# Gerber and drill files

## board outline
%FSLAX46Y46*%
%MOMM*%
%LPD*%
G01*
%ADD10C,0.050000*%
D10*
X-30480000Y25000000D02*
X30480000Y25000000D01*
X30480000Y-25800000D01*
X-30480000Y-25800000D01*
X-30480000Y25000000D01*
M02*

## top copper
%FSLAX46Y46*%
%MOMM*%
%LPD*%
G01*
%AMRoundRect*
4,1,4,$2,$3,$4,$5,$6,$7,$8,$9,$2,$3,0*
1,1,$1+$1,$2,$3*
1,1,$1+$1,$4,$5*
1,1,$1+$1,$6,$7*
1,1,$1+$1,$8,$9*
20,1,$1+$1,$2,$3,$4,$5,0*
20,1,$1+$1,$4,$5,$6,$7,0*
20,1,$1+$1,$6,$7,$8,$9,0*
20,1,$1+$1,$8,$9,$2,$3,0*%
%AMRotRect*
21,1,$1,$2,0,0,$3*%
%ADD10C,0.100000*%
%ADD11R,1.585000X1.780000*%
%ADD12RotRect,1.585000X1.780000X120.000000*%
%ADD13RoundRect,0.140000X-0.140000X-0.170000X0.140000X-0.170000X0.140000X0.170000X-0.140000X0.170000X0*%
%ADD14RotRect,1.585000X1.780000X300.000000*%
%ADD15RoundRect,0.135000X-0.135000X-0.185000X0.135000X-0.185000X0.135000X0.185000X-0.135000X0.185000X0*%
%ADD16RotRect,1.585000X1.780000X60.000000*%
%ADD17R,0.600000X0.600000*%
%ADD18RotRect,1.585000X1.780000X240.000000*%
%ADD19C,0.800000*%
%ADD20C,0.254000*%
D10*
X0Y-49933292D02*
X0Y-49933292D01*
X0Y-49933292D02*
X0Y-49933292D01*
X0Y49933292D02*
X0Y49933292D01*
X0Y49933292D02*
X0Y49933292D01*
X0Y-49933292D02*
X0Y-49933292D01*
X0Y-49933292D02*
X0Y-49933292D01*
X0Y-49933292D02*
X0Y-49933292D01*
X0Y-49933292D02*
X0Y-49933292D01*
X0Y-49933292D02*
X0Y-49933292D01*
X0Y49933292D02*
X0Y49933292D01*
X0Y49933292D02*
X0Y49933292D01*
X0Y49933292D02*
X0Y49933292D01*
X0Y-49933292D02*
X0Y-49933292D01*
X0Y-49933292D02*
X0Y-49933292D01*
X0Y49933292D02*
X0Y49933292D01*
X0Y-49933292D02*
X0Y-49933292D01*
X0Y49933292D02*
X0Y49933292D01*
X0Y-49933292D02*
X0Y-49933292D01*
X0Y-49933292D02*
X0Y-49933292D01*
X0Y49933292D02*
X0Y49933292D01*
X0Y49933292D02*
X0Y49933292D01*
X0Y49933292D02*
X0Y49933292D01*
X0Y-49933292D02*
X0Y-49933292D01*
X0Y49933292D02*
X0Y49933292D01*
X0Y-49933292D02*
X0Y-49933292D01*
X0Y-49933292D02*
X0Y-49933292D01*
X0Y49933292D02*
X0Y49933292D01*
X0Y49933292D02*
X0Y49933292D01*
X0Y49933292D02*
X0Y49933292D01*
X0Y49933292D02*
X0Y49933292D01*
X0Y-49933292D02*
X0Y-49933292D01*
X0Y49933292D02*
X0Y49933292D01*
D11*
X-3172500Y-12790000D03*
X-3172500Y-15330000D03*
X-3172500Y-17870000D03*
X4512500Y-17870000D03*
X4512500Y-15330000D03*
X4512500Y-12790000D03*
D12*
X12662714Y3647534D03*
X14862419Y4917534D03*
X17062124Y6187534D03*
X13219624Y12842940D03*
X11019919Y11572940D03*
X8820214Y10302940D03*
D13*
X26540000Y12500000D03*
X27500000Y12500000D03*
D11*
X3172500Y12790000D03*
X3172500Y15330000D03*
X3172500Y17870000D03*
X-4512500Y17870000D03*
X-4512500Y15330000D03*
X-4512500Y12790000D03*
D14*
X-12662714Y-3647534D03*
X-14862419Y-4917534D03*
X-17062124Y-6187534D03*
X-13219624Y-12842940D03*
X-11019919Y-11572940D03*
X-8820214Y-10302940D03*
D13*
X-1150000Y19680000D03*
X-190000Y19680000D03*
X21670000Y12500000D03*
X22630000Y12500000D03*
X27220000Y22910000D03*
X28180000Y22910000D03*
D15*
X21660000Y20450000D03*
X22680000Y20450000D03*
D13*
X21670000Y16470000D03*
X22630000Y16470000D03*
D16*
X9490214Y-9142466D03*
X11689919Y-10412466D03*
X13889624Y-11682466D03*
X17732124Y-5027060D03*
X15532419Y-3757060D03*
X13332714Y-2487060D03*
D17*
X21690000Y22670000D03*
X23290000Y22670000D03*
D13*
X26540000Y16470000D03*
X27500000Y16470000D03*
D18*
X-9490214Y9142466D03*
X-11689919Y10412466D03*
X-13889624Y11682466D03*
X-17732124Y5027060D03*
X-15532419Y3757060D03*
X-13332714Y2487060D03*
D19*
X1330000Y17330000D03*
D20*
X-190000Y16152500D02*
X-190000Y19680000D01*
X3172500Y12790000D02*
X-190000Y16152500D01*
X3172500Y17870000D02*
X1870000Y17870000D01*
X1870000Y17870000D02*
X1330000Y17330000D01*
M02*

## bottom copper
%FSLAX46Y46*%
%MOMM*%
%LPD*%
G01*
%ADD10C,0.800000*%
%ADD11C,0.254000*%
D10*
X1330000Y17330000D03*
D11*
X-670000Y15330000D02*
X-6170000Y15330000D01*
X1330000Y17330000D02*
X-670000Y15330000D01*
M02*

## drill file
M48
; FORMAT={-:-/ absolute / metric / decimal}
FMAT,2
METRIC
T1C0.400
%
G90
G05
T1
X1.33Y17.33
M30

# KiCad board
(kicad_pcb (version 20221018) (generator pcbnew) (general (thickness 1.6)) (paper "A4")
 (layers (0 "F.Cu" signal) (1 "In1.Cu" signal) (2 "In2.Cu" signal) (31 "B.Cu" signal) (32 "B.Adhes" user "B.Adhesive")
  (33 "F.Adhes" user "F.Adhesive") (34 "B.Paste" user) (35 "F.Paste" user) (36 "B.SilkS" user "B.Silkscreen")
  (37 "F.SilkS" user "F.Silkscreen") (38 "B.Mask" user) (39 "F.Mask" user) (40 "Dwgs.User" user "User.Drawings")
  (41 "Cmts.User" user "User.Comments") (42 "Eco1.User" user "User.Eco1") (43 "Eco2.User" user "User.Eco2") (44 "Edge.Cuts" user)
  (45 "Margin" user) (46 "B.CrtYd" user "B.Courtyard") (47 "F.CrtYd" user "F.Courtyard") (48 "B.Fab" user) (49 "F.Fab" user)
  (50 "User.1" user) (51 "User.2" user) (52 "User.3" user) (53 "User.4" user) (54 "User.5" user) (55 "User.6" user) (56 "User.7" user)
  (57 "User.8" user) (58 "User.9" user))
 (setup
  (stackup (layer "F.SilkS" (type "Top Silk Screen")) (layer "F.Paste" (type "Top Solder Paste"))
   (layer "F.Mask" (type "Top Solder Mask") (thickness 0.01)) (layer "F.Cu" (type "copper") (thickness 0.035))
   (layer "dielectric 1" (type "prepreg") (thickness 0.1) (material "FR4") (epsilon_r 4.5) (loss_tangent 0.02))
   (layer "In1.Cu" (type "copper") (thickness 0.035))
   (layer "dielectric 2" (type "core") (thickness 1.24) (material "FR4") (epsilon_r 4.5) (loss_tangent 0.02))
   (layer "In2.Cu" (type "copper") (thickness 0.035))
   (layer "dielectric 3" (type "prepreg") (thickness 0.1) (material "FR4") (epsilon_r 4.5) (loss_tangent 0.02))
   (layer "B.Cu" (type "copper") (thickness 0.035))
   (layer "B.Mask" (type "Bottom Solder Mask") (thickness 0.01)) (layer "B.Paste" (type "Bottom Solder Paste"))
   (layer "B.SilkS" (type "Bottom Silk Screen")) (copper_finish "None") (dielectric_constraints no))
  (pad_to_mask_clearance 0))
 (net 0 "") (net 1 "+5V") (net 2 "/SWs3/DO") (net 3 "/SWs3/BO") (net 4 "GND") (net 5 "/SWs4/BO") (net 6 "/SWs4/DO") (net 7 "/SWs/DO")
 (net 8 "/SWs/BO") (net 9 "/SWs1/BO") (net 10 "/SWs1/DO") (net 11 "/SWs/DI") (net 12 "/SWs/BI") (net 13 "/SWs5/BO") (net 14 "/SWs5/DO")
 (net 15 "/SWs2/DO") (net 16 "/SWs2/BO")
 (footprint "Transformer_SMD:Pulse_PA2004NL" (layer "F.Cu") (at 0.67 15.33)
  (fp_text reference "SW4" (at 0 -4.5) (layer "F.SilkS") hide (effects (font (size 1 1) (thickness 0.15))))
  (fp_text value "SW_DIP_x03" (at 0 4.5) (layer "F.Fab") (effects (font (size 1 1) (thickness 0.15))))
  (pad "1" smd rect (at -3.8425 -2.54) (size 1.585 1.78) (layers "F.Cu" "F.Paste" "F.Mask") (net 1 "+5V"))
  (pad "2" smd rect (at -3.8425 0) (size 1.585 1.78) (layers "F.Cu" "F.Paste" "F.Mask") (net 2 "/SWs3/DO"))
  (pad "3" smd rect (at -3.8425 2.54) (size 1.585 1.78) (layers "F.Cu" "F.Paste" "F.Mask") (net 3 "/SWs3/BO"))
  (pad "4" smd rect (at 3.8425 2.54) (size 1.585 1.78) (layers "F.Cu" "F.Paste" "F.Mask") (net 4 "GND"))
  (pad "5" smd rect (at 3.8425 0) (size 1.585 1.78) (layers "F.Cu" "F.Paste" "F.Mask") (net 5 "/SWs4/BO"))
  (pad "6" smd rect (at 3.8425 -2.54) (size 1.585 1.78) (layers "F.Cu" "F.Paste" "F.Mask") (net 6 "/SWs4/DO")))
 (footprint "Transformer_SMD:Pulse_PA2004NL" (layer "F.Cu") (at 12.941169 -8.245237 120)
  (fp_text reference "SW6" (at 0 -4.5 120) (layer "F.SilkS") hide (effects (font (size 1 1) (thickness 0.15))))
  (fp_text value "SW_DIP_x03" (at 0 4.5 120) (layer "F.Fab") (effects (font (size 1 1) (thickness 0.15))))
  (pad "1" smd rect (at -3.8425 -2.54 120) (size 1.585 1.78) (layers "F.Cu" "F.Paste" "F.Mask") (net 1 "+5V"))
  (pad "2" smd rect (at -3.8425 0 120) (size 1.585 1.78) (layers "F.Cu" "F.Paste" "F.Mask") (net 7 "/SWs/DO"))
  (pad "3" smd rect (at -3.8425 2.54 120) (size 1.585 1.78) (layers "F.Cu" "F.Paste" "F.Mask") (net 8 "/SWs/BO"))
  (pad "4" smd rect (at 3.8425 2.54 120) (size 1.585 1.78) (layers "F.Cu" "F.Paste" "F.Mask") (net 4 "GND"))
  (pad "5" smd rect (at 3.8425 0 120) (size 1.585 1.78) (layers "F.Cu" "F.Paste" "F.Mask") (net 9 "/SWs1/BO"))
  (pad "6" smd rect (at 3.8425 -2.54 120) (size 1.585 1.78) (layers "F.Cu" "F.Paste" "F.Mask") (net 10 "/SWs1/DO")))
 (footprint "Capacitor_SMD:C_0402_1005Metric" (layer "F.Cu") (at 27.02 -12.5)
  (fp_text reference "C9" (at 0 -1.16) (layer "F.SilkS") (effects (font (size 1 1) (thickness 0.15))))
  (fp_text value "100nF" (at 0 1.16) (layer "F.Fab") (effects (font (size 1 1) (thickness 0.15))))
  (pad "1" smd roundrect (at -0.48 0) (size 0.56 0.62) (layers "F.Cu" "F.Paste" "F.Mask") (roundrect_rratio 0.25) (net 4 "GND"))
  (pad "2" smd roundrect (at 0.48 0) (size 0.56 0.62) (layers "F.Cu" "F.Paste" "F.Mask") (roundrect_rratio 0.25) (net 1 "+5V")))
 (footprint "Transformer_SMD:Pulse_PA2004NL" (layer "F.Cu") (at -0.67 -15.33 180)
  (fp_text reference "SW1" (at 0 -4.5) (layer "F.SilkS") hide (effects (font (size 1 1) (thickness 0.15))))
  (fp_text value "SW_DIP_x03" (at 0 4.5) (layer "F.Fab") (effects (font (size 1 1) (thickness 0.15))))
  (pad "1" smd rect (at -3.8425 -2.54 180) (size 1.585 1.78) (layers "F.Cu" "F.Paste" "F.Mask") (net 1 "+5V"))
  (pad "2" smd rect (at -3.8425 0 180) (size 1.585 1.78) (layers "F.Cu" "F.Paste" "F.Mask") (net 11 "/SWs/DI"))
  (pad "3" smd rect (at -3.8425 2.54 180) (size 1.585 1.78) (layers "F.Cu" "F.Paste" "F.Mask") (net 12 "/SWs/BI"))
  (pad "4" smd rect (at 3.8425 2.54 180) (size 1.585 1.78) (layers "F.Cu" "F.Paste" "F.Mask") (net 4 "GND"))
  (pad "5" smd rect (at 3.8425 0 180) (size 1.585 1.78) (layers "F.Cu" "F.Paste" "F.Mask") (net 8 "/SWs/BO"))
  (pad "6" smd rect (at 3.8425 -2.54 180) (size 1.585 1.78) (layers "F.Cu" "F.Paste" "F.Mask") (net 7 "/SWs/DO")))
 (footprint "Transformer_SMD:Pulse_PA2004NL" (layer "F.Cu") (at -12.941169 8.245237 -60)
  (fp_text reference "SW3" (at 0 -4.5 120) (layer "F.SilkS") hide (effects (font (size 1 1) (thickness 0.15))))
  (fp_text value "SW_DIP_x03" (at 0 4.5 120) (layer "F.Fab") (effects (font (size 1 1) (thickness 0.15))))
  (pad "1" smd rect (at -3.8425 -2.54 300) (size 1.585 1.78) (layers "F.Cu" "F.Paste" "F.Mask") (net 1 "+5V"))
  (pad "2" smd rect (at -3.8425 0 300) (size 1.585 1.78) (layers "F.Cu" "F.Paste" "F.Mask") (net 6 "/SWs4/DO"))
  (pad "3" smd rect (at -3.8425 2.54 300) (size 1.585 1.78) (layers "F.Cu" "F.Paste" "F.Mask") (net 5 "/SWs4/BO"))
  (pad "4" smd rect (at 3.8425 2.54 300) (size 1.585 1.78) (layers "F.Cu" "F.Paste" "F.Mask") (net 4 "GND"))
  (pad "5" smd rect (at 3.8425 0 300) (size 1.585 1.78) (layers "F.Cu" "F.Paste" "F.Mask") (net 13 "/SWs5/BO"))
  (pad "6" smd rect (at 3.8425 -2.54 300) (size 1.585 1.78) (layers "F.Cu" "F.Paste" "F.Mask") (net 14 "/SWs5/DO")))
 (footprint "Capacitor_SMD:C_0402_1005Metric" (layer "F.Cu") (at -0.67 -19.68)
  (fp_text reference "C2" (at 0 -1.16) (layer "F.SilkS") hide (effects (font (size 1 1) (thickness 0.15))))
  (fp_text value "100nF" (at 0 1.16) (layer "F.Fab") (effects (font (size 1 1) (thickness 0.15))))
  (pad "1" smd roundrect (at -0.48 0) (size 0.56 0.62) (layers "F.Cu" "F.Paste" "F.Mask") (roundrect_rratio 0.25) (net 4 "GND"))
  (pad "2" smd roundrect (at 0.48 0) (size 0.56 0.62) (layers "F.Cu" "F.Paste" "F.Mask") (roundrect_rratio 0.25) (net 1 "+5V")))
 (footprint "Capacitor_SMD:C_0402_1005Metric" (layer "F.Cu") (at 22.15 -12.5)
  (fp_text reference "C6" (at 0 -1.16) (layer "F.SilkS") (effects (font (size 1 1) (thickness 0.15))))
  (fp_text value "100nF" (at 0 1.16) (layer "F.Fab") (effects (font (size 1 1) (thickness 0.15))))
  (pad "1" smd roundrect (at -0.48 0) (size 0.56 0.62) (layers "F.Cu" "F.Paste" "F.Mask") (roundrect_rratio 0.25) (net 4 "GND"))
  (pad "2" smd roundrect (at 0.48 0) (size 0.56 0.62) (layers "F.Cu" "F.Paste" "F.Mask") (roundrect_rratio 0.25) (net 1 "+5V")))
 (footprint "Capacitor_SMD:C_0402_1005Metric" (layer "F.Cu") (at 27.7 -22.91)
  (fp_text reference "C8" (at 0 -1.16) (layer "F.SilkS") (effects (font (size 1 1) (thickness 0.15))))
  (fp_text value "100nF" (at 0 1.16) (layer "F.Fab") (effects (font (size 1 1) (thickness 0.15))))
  (pad "1" smd roundrect (at -0.48 0) (size 0.56 0.62) (layers "F.Cu" "F.Paste" "F.Mask") (roundrect_rratio 0.25) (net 4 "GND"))
  (pad "2" smd roundrect (at 0.48 0) (size 0.56 0.62) (layers "F.Cu" "F.Paste" "F.Mask") (roundrect_rratio 0.25) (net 1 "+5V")))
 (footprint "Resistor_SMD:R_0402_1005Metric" (layer "F.Cu") (at 22.17 -20.45)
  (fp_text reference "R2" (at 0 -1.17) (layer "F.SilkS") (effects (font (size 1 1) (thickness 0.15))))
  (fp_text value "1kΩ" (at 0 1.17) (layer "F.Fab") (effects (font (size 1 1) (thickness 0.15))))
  (pad "1" smd roundrect (at -0.51 0) (size 0.54 0.64) (layers "F.Cu" "F.Paste" "F.Mask") (roundrect_rratio 0.25) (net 11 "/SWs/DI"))
  (pad "2" smd roundrect (at 0.51 0) (size 0.54 0.64) (layers "F.Cu" "F.Paste" "F.Mask") (roundrect_rratio 0.25) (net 1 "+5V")))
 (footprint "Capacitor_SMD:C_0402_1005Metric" (layer "F.Cu") (at 22.15 -16.47)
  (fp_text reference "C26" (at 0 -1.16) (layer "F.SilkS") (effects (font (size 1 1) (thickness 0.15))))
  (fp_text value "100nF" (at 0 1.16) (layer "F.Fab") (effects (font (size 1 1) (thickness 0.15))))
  (pad "1" smd roundrect (at -0.48 0) (size 0.56 0.62) (layers "F.Cu" "F.Paste" "F.Mask") (roundrect_rratio 0.25) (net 4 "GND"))
  (pad "2" smd roundrect (at 0.48 0) (size 0.56 0.62) (layers "F.Cu" "F.Paste" "F.Mask") (roundrect_rratio 0.25) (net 1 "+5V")))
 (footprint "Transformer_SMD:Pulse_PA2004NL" (layer "F.Cu") (at 13.611169 7.084763 60)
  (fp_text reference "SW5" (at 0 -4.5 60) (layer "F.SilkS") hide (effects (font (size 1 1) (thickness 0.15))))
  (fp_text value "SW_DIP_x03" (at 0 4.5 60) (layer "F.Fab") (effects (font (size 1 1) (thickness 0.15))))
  (pad "1" smd rect (at -3.8425 -2.54 60) (size 1.585 1.78) (layers "F.Cu" "F.Paste" "F.Mask") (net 1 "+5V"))
  (pad "2" smd rect (at -3.8425 0 60) (size 1.585 1.78) (layers "F.Cu" "F.Paste" "F.Mask") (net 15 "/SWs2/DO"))
  (pad "3" smd rect (at -3.8425 2.54 60) (size 1.585 1.78) (layers "F.Cu" "F.Paste" "F.Mask") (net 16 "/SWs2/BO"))
  (pad "4" smd rect (at 3.8425 2.54 60) (size 1.585 1.78) (layers "F.Cu" "F.Paste" "F.Mask") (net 4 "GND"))
  (pad "5" smd rect (at 3.8425 0 60) (size 1.585 1.78) (layers "F.Cu" "F.Paste" "F.Mask") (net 3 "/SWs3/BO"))
  (pad "6" smd rect (at 3.8425 -2.54 60) (size 1.585 1.78) (layers "F.Cu" "F.Paste" "F.Mask") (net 2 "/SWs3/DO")))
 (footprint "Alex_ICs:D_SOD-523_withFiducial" (layer "F.Cu") (at 22.49 -22.67)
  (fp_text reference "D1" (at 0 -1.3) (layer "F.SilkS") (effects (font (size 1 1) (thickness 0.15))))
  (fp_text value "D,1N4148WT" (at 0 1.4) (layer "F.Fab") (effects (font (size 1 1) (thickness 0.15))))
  (pad "1" smd rect (at -0.8 0 180) (size 0.6 0.6) (layers "F.Cu" "F.Paste" "F.Mask") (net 11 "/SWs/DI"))
  (pad "2" smd rect (at 0.8 0 180) (size 0.6 0.6) (layers "F.Cu" "F.Paste" "F.Mask") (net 4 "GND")))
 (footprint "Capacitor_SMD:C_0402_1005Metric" (layer "F.Cu") (at 27.02 -16.47)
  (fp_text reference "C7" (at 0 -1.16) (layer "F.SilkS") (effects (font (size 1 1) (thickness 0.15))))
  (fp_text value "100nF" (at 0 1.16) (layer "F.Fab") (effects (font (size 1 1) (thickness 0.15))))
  (pad "1" smd roundrect (at -0.48 0) (size 0.56 0.62) (layers "F.Cu" "F.Paste" "F.Mask") (roundrect_rratio 0.25) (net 4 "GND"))
  (pad "2" smd roundrect (at 0.48 0) (size 0.56 0.62) (layers "F.Cu" "F.Paste" "F.Mask") (roundrect_rratio 0.25) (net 1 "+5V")))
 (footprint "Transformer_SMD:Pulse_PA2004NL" (layer "F.Cu") (at -13.611169 -7.084763 -120)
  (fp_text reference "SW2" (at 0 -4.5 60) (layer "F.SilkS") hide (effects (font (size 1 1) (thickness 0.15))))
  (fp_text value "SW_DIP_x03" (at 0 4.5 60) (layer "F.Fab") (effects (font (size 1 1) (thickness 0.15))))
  (pad "1" smd rect (at -3.8425 -2.54 240) (size 1.585 1.78) (layers "F.Cu" "F.Paste" "F.Mask") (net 1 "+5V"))
  (pad "2" smd rect (at -3.8425 0 240) (size 1.585 1.78) (layers "F.Cu" "F.Paste" "F.Mask") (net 10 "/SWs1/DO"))
  (pad "3" smd rect (at -3.8425 2.54 240) (size 1.585 1.78) (layers "F.Cu" "F.Paste" "F.Mask") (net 9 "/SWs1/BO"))
  (pad "4" smd rect (at 3.8425 2.54 240) (size 1.585 1.78) (layers "F.Cu" "F.Paste" "F.Mask") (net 4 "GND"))
  (pad "5" smd rect (at 3.8425 0 240) (size 1.585 1.78) (layers "F.Cu" "F.Paste" "F.Mask") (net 16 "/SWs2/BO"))
  (pad "6" smd rect (at 3.8425 -2.54 240) (size 1.585 1.78) (layers "F.Cu" "F.Paste" "F.Mask") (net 15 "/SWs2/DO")))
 (gr_line (start 0 49.933292) (end 0 49.933292) (stroke (width 0.1) (type default)) (layer "F.Cu"))
 (gr_line (start 0 49.933292) (end 0 49.933292) (stroke (width 0.1) (type default)) (layer "F.Cu"))
 (gr_line (start 0 -49.933292) (end 0 -49.933292) (stroke (width 0.1) (type default)) (layer "F.Cu"))
 (gr_line (start 0 -49.933292) (end 0 -49.933292) (stroke (width 0.1) (type default)) (layer "F.Cu"))
 (gr_line (start 0 49.933292) (end 0 49.933292) (stroke (width 0.1) (type default)) (layer "F.Cu"))
 (gr_line (start 0 49.933292) (end 0 49.933292) (stroke (width 0.1) (type default)) (layer "F.Cu"))
 (gr_line (start 0 49.933292) (end 0 49.933292) (stroke (width 0.1) (type default)) (layer "F.Cu"))
 (gr_line (start 0 49.933292) (end 0 49.933292) (stroke (width 0.1) (type default)) (layer "F.Cu"))
 (gr_line (start 0 49.933292) (end 0 49.933292) (stroke (width 0.1) (type default)) (layer "F.Cu"))
 (gr_line (start 0 -49.933292) (end 0 -49.933292) (stroke (width 0.1) (type default)) (layer "F.Cu"))
 (gr_line (start 0 -49.933292) (end 0 -49.933292) (stroke (width 0.1) (type default)) (layer "F.Cu"))
 (gr_line (start 0 -49.933292) (end 0 -49.933292) (stroke (width 0.1) (type default)) (layer "F.Cu"))
 (gr_line (start 0 49.933292) (end 0 49.933292) (stroke (width 0.1) (type default)) (layer "F.Cu"))
 (gr_line (start 0 49.933292) (end 0 49.933292) (stroke (width 0.1) (type default)) (layer "F.Cu"))
 (gr_line (start 0 -49.933292) (end 0 -49.933292) (stroke (width 0.1) (type default)) (layer "F.Cu"))
 (gr_line (start 0 49.933292) (end 0 49.933292) (stroke (width 0.1) (type default)) (layer "F.Cu"))
 (gr_line (start 0 -49.933292) (end 0 -49.933292) (stroke (width 0.1) (type default)) (layer "F.Cu"))
 (gr_line (start 0 49.933292) (end 0 49.933292) (stroke (width 0.1) (type default)) (layer "F.Cu"))
 (gr_line (start 0 49.933292) (end 0 49.933292) (stroke (width 0.1) (type default)) (layer "F.Cu"))
 (gr_line (start 0 -49.933292) (end 0 -49.933292) (stroke (width 0.1) (type default)) (layer "F.Cu"))
 (gr_line (start 0 -49.933292) (end 0 -49.933292) (stroke (width 0.1) (type default)) (layer "F.Cu"))
 (gr_line (start 0 -49.933292) (end 0 -49.933292) (stroke (width 0.1) (type default)) (layer "F.Cu"))
 (gr_line (start 0 49.933292) (end 0 49.933292) (stroke (width 0.1) (type default)) (layer "F.Cu"))
 (gr_line (start 0 -49.933292) (end 0 -49.933292) (stroke (width 0.1) (type default)) (layer "F.Cu"))
 (gr_line (start 0 49.933292) (end 0 49.933292) (stroke (width 0.1) (type default)) (layer "F.Cu"))
 (gr_line (start 0 49.933292) (end 0 49.933292) (stroke (width 0.1) (type default)) (layer "F.Cu"))
 (gr_line (start 0 -49.933292) (end 0 -49.933292) (stroke (width 0.1) (type default)) (layer "F.Cu"))
 (gr_line (start 0 -49.933292) (end 0 -49.933292) (stroke (width 0.1) (type default)) (layer "F.Cu"))
 (gr_line (start 0 -49.933292) (end 0 -49.933292) (stroke (width 0.1) (type default)) (layer "F.Cu"))
 (gr_line (start 0 -49.933292) (end 0 -49.933292) (stroke (width 0.1) (type default)) (layer "F.Cu"))
 (gr_line (start 0 49.933292) (end 0 49.933292) (stroke (width 0.1) (type default)) (layer "F.Cu"))
 (gr_line (start 0 -49.933292) (end 0 -49.933292) (stroke (width 0.1) (type default)) (layer "F.Cu"))
 (gr_rect (start -30.48 -25) (end 30.48 25.8) (stroke (width 0.05) (type default)) (fill none) (layer "Edge.Cuts"))
 (segment (start -0.19 -16.1525) (end -0.19 -19.68) (width 0.254) (layer "F.Cu") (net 1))
 (segment (start 3.1725 -12.79) (end -0.19 -16.1525) (width 0.254) (layer "F.Cu") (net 1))
 (segment (start 3.1725 -17.87) (end 1.87 -17.87) (width 0.254) (layer "F.Cu") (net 12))
 (segment (start 1.87 -17.87) (end 1.33 -17.33) (width 0.254) (layer "F.Cu") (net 12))
 (via (at 1.33 -17.33) (size 0.8) (drill 0.4) (layers "F.Cu" "B.Cu") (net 12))
 (segment (start -0.67 -15.33) (end -6.17 -15.33) (width 0.254) (layer "B.Cu") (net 12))
 (segment (start 1.33 -17.33) (end -0.67 -15.33) (width 0.254) (layer "B.Cu") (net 12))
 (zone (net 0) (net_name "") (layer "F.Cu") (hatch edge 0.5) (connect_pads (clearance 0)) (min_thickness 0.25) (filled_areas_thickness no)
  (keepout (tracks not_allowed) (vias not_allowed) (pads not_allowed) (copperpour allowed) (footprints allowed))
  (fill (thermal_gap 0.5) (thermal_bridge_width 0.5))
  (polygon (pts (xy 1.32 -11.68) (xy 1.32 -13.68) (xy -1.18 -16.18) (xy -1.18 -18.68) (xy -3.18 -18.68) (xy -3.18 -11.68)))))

